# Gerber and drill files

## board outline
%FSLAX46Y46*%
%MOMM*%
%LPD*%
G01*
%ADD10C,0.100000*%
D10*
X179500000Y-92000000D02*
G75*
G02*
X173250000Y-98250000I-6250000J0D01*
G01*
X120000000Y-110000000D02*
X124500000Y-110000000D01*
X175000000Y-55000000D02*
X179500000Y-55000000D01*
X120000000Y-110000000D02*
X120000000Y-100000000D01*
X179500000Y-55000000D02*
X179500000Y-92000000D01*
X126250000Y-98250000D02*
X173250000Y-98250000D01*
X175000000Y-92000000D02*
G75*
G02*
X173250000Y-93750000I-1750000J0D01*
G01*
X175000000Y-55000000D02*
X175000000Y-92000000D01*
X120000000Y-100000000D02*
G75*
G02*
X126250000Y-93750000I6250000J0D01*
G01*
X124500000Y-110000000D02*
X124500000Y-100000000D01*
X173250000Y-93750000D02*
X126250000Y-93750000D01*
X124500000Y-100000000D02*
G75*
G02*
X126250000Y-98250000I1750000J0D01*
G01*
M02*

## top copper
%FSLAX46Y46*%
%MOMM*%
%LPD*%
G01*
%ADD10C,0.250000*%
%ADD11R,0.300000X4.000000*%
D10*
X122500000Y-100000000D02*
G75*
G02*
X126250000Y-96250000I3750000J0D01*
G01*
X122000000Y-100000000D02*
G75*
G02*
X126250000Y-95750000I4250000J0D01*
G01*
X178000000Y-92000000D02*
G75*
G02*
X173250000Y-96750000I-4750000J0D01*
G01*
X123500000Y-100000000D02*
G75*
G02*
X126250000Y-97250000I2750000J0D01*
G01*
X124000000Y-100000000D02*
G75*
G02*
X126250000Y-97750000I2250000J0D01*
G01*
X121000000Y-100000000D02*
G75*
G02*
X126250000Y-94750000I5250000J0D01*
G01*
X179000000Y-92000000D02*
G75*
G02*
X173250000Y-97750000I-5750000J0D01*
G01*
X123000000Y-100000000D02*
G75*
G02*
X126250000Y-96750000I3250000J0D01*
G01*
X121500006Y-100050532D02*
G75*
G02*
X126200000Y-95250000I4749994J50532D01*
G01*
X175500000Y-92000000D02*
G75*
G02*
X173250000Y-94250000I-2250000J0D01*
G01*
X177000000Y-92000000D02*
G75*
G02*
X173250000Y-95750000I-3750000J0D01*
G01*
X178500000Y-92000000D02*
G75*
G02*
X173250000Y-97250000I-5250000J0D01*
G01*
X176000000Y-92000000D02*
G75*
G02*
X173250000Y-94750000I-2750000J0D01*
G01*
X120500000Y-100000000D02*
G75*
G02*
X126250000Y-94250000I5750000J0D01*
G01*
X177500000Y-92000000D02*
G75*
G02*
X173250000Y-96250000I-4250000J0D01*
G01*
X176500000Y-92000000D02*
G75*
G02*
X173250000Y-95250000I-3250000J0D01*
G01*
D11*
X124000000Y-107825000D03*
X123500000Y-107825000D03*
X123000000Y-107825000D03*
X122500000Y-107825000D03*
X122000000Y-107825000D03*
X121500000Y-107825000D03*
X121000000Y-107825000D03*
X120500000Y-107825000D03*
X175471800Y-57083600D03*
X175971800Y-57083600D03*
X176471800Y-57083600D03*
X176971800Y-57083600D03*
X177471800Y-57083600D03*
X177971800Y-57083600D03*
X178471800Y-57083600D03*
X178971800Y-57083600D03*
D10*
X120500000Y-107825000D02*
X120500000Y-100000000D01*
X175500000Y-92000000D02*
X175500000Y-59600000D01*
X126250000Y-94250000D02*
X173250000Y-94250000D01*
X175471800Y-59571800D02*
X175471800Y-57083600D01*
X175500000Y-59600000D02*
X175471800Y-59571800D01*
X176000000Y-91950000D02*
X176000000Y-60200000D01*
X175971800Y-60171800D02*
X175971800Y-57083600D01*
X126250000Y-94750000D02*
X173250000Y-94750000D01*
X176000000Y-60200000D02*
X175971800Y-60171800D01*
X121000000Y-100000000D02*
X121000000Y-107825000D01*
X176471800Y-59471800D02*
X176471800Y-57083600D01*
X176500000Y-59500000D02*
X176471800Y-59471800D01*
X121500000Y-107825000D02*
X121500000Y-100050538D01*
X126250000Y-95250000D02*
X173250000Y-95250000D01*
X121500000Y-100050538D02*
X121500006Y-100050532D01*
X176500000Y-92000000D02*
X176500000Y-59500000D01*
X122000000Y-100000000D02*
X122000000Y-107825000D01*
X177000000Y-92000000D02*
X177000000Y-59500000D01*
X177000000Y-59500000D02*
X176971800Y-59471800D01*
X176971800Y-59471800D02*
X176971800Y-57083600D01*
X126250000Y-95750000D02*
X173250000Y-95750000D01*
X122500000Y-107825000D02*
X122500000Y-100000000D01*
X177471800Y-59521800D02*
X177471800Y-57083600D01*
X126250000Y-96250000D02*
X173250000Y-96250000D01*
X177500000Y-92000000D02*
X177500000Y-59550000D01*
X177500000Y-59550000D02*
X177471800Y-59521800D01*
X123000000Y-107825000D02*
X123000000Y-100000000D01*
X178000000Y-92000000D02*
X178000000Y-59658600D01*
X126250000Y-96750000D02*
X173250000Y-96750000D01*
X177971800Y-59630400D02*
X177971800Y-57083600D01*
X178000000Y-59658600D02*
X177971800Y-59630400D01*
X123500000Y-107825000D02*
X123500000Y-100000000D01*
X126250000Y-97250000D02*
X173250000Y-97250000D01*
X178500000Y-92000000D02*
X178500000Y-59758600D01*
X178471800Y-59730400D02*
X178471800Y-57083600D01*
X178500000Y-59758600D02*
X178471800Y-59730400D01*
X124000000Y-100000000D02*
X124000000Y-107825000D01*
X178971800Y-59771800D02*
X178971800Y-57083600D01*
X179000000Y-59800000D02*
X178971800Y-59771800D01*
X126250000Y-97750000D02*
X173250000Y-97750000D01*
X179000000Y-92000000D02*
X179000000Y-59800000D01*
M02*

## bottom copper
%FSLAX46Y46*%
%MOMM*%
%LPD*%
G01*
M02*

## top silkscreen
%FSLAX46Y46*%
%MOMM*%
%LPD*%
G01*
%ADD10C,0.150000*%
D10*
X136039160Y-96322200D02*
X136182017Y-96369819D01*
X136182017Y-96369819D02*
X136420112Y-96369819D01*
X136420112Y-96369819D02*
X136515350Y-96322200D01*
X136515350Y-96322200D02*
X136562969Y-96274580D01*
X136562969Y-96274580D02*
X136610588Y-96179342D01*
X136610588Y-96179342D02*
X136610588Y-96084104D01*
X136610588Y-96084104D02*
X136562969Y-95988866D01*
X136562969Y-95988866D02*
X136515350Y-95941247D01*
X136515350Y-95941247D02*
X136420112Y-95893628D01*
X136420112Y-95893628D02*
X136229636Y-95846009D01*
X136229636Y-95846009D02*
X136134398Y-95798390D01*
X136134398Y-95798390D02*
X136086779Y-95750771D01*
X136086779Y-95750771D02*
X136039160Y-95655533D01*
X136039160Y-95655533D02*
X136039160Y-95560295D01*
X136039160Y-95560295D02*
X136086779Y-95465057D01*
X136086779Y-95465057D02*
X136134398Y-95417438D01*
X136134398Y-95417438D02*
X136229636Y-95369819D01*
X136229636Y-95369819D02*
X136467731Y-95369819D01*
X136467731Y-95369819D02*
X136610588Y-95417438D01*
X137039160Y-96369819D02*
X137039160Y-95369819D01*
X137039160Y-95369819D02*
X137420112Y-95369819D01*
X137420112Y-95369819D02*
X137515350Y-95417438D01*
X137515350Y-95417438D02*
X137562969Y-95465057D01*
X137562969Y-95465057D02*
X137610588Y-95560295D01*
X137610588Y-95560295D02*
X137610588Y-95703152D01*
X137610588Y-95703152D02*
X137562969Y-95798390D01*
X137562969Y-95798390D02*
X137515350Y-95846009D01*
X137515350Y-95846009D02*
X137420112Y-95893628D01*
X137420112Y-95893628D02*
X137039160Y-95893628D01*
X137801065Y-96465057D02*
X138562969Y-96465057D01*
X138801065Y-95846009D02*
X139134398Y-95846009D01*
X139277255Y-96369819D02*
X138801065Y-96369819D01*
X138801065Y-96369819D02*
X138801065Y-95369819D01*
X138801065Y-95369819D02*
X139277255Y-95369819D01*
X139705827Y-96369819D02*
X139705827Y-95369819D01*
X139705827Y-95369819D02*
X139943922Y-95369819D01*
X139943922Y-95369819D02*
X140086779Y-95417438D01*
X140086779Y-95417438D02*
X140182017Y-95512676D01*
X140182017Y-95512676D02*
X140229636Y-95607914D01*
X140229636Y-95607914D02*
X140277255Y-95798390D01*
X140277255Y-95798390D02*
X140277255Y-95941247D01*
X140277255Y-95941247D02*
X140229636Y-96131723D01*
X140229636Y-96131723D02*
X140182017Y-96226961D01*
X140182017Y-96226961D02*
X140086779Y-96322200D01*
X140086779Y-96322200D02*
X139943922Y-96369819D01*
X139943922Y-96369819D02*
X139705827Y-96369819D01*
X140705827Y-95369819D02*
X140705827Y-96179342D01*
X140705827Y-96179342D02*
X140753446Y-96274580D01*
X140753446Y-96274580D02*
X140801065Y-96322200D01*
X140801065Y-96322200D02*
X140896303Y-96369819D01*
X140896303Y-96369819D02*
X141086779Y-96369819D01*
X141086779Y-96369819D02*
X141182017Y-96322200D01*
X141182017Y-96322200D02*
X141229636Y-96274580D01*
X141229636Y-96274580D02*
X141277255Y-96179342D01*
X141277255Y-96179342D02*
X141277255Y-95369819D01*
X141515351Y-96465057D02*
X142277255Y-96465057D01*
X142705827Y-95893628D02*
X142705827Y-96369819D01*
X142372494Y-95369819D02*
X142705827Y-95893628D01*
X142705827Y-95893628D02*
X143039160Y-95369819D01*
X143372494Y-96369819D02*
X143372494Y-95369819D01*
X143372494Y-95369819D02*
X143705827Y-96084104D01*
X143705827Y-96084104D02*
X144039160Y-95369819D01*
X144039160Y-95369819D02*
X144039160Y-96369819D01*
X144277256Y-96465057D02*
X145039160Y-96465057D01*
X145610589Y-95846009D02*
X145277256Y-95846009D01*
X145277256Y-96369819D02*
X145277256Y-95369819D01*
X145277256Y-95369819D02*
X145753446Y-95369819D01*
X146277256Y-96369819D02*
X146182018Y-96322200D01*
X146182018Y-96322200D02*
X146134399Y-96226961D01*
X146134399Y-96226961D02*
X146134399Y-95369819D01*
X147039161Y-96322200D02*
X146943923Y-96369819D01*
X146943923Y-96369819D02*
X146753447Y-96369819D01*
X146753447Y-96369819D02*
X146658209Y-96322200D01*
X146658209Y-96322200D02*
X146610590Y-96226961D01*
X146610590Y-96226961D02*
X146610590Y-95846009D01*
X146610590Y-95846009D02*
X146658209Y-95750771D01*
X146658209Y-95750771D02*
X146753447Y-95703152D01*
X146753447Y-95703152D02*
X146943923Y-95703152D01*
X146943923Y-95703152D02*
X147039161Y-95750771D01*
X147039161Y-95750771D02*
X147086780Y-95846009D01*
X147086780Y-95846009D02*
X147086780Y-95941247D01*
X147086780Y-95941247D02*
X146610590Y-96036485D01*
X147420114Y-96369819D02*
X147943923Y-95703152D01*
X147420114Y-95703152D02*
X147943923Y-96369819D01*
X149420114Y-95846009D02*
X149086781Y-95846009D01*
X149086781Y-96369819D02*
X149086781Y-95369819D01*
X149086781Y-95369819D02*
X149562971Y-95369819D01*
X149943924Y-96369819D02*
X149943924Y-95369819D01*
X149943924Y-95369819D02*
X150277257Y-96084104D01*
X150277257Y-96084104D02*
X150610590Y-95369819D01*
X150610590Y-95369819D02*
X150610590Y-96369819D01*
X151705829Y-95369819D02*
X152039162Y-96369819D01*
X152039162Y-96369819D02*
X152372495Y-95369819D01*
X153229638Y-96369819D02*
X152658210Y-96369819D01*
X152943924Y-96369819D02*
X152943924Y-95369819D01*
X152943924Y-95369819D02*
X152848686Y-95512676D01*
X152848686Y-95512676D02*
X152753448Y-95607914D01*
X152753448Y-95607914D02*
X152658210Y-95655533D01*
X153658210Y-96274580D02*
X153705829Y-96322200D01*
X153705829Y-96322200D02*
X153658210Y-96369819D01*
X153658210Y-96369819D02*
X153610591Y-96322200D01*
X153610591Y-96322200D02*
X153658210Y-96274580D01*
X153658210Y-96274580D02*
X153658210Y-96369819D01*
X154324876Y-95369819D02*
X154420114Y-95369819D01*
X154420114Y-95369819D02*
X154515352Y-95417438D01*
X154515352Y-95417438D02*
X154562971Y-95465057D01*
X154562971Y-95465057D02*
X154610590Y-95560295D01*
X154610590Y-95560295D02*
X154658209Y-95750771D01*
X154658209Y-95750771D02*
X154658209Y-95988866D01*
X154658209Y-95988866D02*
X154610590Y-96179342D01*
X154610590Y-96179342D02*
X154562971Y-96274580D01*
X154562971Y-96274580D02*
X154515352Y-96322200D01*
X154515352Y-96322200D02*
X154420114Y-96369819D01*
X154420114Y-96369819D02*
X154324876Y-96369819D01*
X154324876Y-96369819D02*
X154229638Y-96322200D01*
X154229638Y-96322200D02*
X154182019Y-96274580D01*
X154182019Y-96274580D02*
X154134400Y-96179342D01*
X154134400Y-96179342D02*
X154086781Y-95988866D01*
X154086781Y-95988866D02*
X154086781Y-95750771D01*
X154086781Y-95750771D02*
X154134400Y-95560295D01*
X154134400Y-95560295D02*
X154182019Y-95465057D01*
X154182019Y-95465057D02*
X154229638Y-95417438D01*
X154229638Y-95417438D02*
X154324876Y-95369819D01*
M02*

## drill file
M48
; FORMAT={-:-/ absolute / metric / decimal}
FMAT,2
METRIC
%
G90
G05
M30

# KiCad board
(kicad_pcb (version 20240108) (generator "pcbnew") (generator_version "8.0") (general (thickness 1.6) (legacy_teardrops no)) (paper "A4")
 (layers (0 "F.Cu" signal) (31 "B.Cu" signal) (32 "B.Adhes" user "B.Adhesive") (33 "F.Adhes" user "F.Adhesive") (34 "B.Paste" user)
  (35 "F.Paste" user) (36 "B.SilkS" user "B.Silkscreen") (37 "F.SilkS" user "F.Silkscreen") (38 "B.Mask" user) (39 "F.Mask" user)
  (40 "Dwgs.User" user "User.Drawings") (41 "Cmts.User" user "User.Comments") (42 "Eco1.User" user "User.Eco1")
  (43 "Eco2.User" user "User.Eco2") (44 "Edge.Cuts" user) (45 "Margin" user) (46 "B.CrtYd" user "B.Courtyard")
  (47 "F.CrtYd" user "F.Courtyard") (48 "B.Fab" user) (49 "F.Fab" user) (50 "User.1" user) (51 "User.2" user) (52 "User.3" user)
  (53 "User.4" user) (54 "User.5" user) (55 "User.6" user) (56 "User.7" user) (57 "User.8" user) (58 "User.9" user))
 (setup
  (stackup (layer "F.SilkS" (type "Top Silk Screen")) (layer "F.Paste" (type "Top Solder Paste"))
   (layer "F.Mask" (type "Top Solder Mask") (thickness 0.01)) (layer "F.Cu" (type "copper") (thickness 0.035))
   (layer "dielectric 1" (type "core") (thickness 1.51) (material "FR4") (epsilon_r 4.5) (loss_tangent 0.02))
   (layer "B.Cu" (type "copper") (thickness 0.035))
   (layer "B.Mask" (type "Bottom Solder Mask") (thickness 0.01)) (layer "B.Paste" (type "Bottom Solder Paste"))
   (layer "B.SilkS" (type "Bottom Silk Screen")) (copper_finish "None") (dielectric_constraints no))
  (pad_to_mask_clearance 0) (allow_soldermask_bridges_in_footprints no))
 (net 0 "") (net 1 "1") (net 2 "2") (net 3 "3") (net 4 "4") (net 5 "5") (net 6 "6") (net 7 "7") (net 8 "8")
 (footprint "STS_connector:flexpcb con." (layer "F.Cu") (at 124.5 105.825 180)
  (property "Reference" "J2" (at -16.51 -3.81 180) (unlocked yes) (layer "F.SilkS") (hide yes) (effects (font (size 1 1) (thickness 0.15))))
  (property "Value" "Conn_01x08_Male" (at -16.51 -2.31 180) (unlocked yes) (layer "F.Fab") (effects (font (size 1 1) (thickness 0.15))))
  (pad "1" smd rect (at 0.5 -2 180) (size 0.3 4) (layers "F.Cu" "F.Paste" "F.Mask") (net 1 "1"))
  (pad "2" smd rect (at 1 -2 180) (size 0.3 4) (layers "F.Cu" "F.Paste" "F.Mask") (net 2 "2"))
  (pad "3" smd rect (at 1.5 -2 180) (size 0.3 4) (layers "F.Cu" "F.Paste" "F.Mask") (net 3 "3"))
  (pad "4" smd rect (at 2 -2 180) (size 0.3 4) (layers "F.Cu" "F.Paste" "F.Mask") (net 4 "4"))
  (pad "5" smd rect (at 2.5 -2 180) (size 0.3 4) (layers "F.Cu" "F.Paste" "F.Mask") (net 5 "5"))
  (pad "6" smd rect (at 3 -2 180) (size 0.3 4) (layers "F.Cu" "F.Paste" "F.Mask") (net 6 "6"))
  (pad "7" smd rect (at 3.5 -2 180) (size 0.3 4) (layers "F.Cu" "F.Paste" "F.Mask") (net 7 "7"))
  (pad "8" smd rect (at 4 -2 180) (size 0.3 4) (layers "F.Cu" "F.Paste" "F.Mask") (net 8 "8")))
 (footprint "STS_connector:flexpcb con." (layer "F.Cu") (at 174.9718 59.0836)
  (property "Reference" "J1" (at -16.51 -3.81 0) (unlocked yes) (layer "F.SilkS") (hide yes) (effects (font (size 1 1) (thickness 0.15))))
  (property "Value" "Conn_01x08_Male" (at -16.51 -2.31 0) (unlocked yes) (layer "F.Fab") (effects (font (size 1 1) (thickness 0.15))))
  (pad "1" smd rect (at 0.5 -2) (size 0.3 4) (layers "F.Cu" "F.Paste" "F.Mask") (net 8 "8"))
  (pad "2" smd rect (at 1 -2) (size 0.3 4) (layers "F.Cu" "F.Paste" "F.Mask") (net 7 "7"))
  (pad "3" smd rect (at 1.5 -2) (size 0.3 4) (layers "F.Cu" "F.Paste" "F.Mask") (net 6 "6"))
  (pad "4" smd rect (at 2 -2) (size 0.3 4) (layers "F.Cu" "F.Paste" "F.Mask") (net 5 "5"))
  (pad "5" smd rect (at 2.5 -2) (size 0.3 4) (layers "F.Cu" "F.Paste" "F.Mask") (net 4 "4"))
  (pad "6" smd rect (at 3 -2) (size 0.3 4) (layers "F.Cu" "F.Paste" "F.Mask") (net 3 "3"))
  (pad "7" smd rect (at 3.5 -2) (size 0.3 4) (layers "F.Cu" "F.Paste" "F.Mask") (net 2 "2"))
  (pad "8" smd rect (at 4 -2) (size 0.3 4) (layers "F.Cu" "F.Paste" "F.Mask") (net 1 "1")))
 (gr_arc (start 122.5 100) (mid 123.59835 97.34835) (end 126.25 96.25) (stroke (width 0.25) (type default)) (layer "F.Cu") (net 4))
 (gr_arc (start 122 100) (mid 123.244796 96.994796) (end 126.25 95.75) (stroke (width 0.25) (type default)) (layer "F.Cu") (net 5))
 (gr_arc (start 178 92) (mid 176.608757 95.358757) (end 173.25 96.75) (stroke (width 0.25) (type default)) (layer "F.Cu") (net 3))
 (gr_arc (start 123.5 100) (mid 124.305456 98.055456) (end 126.25 97.25) (stroke (width 0.25) (type default)) (layer "F.Cu") (net 2))
 (gr_arc (start 124 100) (mid 124.65901 98.40901) (end 126.25 97.75) (stroke (width 0.25) (type default)) (layer "F.Cu") (net 1))
 (gr_arc (start 121 100) (mid 122.537689 96.287689) (end 126.25 94.75) (stroke (width 0.25) (type default)) (layer "F.Cu") (net 7))
 (gr_arc (start 179 92) (mid 177.315864 96.065864) (end 173.25 97.75) (stroke (width 0.25) (type default)) (layer "F.Cu") (net 1))
 (gr_arc (start 123 100) (mid 123.951903 97.701903) (end 126.25 96.75) (stroke (width 0.25) (type default)) (layer "F.Cu") (net 3))
 (gr_arc (start 121.500006 100.050532) (mid 122.855701 96.676788) (end 126.2 95.25) (stroke (width 0.25) (type default)) (layer "F.Cu")
  (net 6))
 (gr_arc (start 175.5 92) (mid 174.84099 93.59099) (end 173.25 94.25) (stroke (width 0.25) (type default)) (layer "F.Cu") (net 8))
 (gr_arc (start 177 92) (mid 175.90165 94.65165) (end 173.25 95.75) (stroke (width 0.25) (type default)) (layer "F.Cu") (net 5))
 (gr_arc (start 178.5 92) (mid 176.962311 95.712311) (end 173.25 97.25) (stroke (width 0.25) (type default)) (layer "F.Cu") (net 2))
 (gr_arc (start 176 92) (mid 175.194544 93.944544) (end 173.25 94.75) (stroke (width 0.25) (type default)) (layer "F.Cu") (net 7))
 (gr_arc (start 120.5 100) (mid 122.184136 95.934136) (end 126.25 94.25) (stroke (width 0.25) (type default)) (layer "F.Cu") (net 8))
 (gr_arc (start 177.5 92) (mid 176.255204 95.005204) (end 173.25 96.25) (stroke (width 0.25) (type default)) (layer "F.Cu") (net 4))
 (gr_arc (start 176.5 92) (mid 175.548097 94.298097) (end 173.25 95.25) (stroke (width 0.25) (type default)) (layer "F.Cu") (net 6))
 (gr_arc (start 179.5 92) (mid 177.669417 96.419417) (end 173.25 98.25) (stroke (width 0.1) (type default)) (layer "Edge.Cuts"))
 (gr_line (start 120 110) (end 124.5 110) (stroke (width 0.1) (type solid)) (layer "Edge.Cuts"))
 (gr_line (start 175 55) (end 179.5 55) (stroke (width 0.1) (type default)) (layer "Edge.Cuts"))
 (gr_line (start 120 110) (end 120 100) (stroke (width 0.1) (type default)) (layer "Edge.Cuts"))
 (gr_line (start 179.5 55) (end 179.5 92) (stroke (width 0.1) (type default)) (layer "Edge.Cuts"))
 (gr_line (start 126.25 98.25) (end 173.25 98.25) (stroke (width 0.1) (type default)) (layer "Edge.Cuts"))
 (gr_arc (start 175 92) (mid 174.487437 93.237437) (end 173.25 93.75) (stroke (width 0.1) (type default)) (layer "Edge.Cuts"))
 (gr_line (start 175 55) (end 175 92) (stroke (width 0.1) (type default)) (layer "Edge.Cuts"))
 (gr_arc (start 120 100) (mid 121.830583 95.580583) (end 126.25 93.75) (stroke (width 0.1) (type default)) (layer "Edge.Cuts"))
 (gr_line (start 124.5 110) (end 124.5 100) (stroke (width 0.1) (type default)) (layer "Edge.Cuts"))
 (gr_line (start 173.25 93.75) (end 126.25 93.75) (stroke (width 0.1) (type default)) (layer "Edge.Cuts"))
 (gr_arc (start 124.5 100) (mid 125.012563 98.762563) (end 126.25 98.25) (stroke (width 0.1) (type default)) (layer "Edge.Cuts"))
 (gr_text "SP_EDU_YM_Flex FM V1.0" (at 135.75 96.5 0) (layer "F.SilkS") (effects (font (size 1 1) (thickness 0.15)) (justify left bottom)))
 (segment (start 120.5 107.825) (end 120.5 100) (width 0.25) (layer "F.Cu") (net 8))
 (segment (start 175.5 92) (end 175.5 59.6) (width 0.25) (layer "F.Cu") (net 8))
 (segment (start 126.25 94.25) (end 173.25 94.25) (width 0.25) (layer "F.Cu") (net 8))
 (segment (start 175.4718 59.5718) (end 175.4718 57.0836) (width 0.25) (layer "F.Cu") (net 8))
 (segment (start 175.5 59.6) (end 175.4718 59.5718) (width 0.25) (layer "F.Cu") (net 8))
 (segment (start 176 91.95) (end 176 60.2) (width 0.25) (layer "F.Cu") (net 7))
 (segment (start 175.9718 60.1718) (end 175.9718 57.0836) (width 0.25) (layer "F.Cu") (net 7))
 (segment (start 126.25 94.75) (end 173.25 94.75) (width 0.25) (layer "F.Cu") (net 7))
 (segment (start 176 60.2) (end 175.9718 60.1718) (width 0.25) (layer "F.Cu") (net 7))
 (segment (start 121 100) (end 121 107.825) (width 0.25) (layer "F.Cu") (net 7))
 (segment (start 176.4718 59.4718) (end 176.4718 57.0836) (width 0.25) (layer "F.Cu") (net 6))
 (segment (start 176.5 59.5) (end 176.4718 59.4718) (width 0.25) (layer "F.Cu") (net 6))
 (segment (start 121.5 107.825) (end 121.5 100.050538) (width 0.25) (layer "F.Cu") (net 6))
 (segment (start 126.25 95.25) (end 173.25 95.25) (width 0.25) (layer "F.Cu") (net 6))
 (segment (start 121.5 100.050538) (end 121.500006 100.050532) (width 0.25) (layer "F.Cu") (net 6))
 (segment (start 176.5 92) (end 176.5 59.5) (width 0.25) (layer "F.Cu") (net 6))
 (segment (start 122 100) (end 122 107.825) (width 0.25) (layer "F.Cu") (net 5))
 (segment (start 177 92) (end 177 59.5) (width 0.25) (layer "F.Cu") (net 5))
 (segment (start 177 59.5) (end 176.9718 59.4718) (width 0.25) (layer "F.Cu") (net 5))
 (segment (start 176.9718 59.4718) (end 176.9718 57.0836) (width 0.25) (layer "F.Cu") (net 5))
 (segment (start 126.25 95.75) (end 173.25 95.75) (width 0.25) (layer "F.Cu") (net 5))
 (segment (start 122.5 107.825) (end 122.5 100) (width 0.25) (layer "F.Cu") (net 4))
 (segment (start 177.4718 59.5218) (end 177.4718 57.0836) (width 0.25) (layer "F.Cu") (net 4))
 (segment (start 126.25 96.25) (end 173.25 96.25) (width 0.25) (layer "F.Cu") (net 4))
 (segment (start 177.5 92) (end 177.5 59.55) (width 0.25) (layer "F.Cu") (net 4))
 (segment (start 177.5 59.55) (end 177.4718 59.5218) (width 0.25) (layer "F.Cu") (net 4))
 (segment (start 123 107.825) (end 123 100) (width 0.25) (layer "F.Cu") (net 3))
 (segment (start 178 92) (end 178 59.6586) (width 0.25) (layer "F.Cu") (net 3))
 (segment (start 126.25 96.75) (end 173.25 96.75) (width 0.25) (layer "F.Cu") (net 3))
 (segment (start 177.9718 59.6304) (end 177.9718 57.0836) (width 0.25) (layer "F.Cu") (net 3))
 (segment (start 178 59.6586) (end 177.9718 59.6304) (width 0.25) (layer "F.Cu") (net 3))
 (segment (start 123.5 107.825) (end 123.5 100) (width 0.25) (layer "F.Cu") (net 2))
 (segment (start 126.25 97.25) (end 173.25 97.25) (width 0.25) (layer "F.Cu") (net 2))
 (segment (start 178.5 92) (end 178.5 59.7586) (width 0.25) (layer "F.Cu") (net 2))
 (segment (start 178.4718 59.7304) (end 178.4718 57.0836) (width 0.25) (layer "F.Cu") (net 2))
 (segment (start 178.5 59.7586) (end 178.4718 59.7304) (width 0.25) (layer "F.Cu") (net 2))
 (segment (start 124 100) (end 124 107.825) (width 0.25) (layer "F.Cu") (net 1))
 (segment (start 178.9718 59.7718) (end 178.9718 57.0836) (width 0.25) (layer "F.Cu") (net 1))
 (segment (start 179 59.8) (end 178.9718 59.7718) (width 0.25) (layer "F.Cu") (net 1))
 (segment (start 126.25 97.75) (end 173.25 97.75) (width 0.25) (layer "F.Cu") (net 1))
 (segment (start 179 92) (end 179 59.8) (width 0.25) (layer "F.Cu") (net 1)))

